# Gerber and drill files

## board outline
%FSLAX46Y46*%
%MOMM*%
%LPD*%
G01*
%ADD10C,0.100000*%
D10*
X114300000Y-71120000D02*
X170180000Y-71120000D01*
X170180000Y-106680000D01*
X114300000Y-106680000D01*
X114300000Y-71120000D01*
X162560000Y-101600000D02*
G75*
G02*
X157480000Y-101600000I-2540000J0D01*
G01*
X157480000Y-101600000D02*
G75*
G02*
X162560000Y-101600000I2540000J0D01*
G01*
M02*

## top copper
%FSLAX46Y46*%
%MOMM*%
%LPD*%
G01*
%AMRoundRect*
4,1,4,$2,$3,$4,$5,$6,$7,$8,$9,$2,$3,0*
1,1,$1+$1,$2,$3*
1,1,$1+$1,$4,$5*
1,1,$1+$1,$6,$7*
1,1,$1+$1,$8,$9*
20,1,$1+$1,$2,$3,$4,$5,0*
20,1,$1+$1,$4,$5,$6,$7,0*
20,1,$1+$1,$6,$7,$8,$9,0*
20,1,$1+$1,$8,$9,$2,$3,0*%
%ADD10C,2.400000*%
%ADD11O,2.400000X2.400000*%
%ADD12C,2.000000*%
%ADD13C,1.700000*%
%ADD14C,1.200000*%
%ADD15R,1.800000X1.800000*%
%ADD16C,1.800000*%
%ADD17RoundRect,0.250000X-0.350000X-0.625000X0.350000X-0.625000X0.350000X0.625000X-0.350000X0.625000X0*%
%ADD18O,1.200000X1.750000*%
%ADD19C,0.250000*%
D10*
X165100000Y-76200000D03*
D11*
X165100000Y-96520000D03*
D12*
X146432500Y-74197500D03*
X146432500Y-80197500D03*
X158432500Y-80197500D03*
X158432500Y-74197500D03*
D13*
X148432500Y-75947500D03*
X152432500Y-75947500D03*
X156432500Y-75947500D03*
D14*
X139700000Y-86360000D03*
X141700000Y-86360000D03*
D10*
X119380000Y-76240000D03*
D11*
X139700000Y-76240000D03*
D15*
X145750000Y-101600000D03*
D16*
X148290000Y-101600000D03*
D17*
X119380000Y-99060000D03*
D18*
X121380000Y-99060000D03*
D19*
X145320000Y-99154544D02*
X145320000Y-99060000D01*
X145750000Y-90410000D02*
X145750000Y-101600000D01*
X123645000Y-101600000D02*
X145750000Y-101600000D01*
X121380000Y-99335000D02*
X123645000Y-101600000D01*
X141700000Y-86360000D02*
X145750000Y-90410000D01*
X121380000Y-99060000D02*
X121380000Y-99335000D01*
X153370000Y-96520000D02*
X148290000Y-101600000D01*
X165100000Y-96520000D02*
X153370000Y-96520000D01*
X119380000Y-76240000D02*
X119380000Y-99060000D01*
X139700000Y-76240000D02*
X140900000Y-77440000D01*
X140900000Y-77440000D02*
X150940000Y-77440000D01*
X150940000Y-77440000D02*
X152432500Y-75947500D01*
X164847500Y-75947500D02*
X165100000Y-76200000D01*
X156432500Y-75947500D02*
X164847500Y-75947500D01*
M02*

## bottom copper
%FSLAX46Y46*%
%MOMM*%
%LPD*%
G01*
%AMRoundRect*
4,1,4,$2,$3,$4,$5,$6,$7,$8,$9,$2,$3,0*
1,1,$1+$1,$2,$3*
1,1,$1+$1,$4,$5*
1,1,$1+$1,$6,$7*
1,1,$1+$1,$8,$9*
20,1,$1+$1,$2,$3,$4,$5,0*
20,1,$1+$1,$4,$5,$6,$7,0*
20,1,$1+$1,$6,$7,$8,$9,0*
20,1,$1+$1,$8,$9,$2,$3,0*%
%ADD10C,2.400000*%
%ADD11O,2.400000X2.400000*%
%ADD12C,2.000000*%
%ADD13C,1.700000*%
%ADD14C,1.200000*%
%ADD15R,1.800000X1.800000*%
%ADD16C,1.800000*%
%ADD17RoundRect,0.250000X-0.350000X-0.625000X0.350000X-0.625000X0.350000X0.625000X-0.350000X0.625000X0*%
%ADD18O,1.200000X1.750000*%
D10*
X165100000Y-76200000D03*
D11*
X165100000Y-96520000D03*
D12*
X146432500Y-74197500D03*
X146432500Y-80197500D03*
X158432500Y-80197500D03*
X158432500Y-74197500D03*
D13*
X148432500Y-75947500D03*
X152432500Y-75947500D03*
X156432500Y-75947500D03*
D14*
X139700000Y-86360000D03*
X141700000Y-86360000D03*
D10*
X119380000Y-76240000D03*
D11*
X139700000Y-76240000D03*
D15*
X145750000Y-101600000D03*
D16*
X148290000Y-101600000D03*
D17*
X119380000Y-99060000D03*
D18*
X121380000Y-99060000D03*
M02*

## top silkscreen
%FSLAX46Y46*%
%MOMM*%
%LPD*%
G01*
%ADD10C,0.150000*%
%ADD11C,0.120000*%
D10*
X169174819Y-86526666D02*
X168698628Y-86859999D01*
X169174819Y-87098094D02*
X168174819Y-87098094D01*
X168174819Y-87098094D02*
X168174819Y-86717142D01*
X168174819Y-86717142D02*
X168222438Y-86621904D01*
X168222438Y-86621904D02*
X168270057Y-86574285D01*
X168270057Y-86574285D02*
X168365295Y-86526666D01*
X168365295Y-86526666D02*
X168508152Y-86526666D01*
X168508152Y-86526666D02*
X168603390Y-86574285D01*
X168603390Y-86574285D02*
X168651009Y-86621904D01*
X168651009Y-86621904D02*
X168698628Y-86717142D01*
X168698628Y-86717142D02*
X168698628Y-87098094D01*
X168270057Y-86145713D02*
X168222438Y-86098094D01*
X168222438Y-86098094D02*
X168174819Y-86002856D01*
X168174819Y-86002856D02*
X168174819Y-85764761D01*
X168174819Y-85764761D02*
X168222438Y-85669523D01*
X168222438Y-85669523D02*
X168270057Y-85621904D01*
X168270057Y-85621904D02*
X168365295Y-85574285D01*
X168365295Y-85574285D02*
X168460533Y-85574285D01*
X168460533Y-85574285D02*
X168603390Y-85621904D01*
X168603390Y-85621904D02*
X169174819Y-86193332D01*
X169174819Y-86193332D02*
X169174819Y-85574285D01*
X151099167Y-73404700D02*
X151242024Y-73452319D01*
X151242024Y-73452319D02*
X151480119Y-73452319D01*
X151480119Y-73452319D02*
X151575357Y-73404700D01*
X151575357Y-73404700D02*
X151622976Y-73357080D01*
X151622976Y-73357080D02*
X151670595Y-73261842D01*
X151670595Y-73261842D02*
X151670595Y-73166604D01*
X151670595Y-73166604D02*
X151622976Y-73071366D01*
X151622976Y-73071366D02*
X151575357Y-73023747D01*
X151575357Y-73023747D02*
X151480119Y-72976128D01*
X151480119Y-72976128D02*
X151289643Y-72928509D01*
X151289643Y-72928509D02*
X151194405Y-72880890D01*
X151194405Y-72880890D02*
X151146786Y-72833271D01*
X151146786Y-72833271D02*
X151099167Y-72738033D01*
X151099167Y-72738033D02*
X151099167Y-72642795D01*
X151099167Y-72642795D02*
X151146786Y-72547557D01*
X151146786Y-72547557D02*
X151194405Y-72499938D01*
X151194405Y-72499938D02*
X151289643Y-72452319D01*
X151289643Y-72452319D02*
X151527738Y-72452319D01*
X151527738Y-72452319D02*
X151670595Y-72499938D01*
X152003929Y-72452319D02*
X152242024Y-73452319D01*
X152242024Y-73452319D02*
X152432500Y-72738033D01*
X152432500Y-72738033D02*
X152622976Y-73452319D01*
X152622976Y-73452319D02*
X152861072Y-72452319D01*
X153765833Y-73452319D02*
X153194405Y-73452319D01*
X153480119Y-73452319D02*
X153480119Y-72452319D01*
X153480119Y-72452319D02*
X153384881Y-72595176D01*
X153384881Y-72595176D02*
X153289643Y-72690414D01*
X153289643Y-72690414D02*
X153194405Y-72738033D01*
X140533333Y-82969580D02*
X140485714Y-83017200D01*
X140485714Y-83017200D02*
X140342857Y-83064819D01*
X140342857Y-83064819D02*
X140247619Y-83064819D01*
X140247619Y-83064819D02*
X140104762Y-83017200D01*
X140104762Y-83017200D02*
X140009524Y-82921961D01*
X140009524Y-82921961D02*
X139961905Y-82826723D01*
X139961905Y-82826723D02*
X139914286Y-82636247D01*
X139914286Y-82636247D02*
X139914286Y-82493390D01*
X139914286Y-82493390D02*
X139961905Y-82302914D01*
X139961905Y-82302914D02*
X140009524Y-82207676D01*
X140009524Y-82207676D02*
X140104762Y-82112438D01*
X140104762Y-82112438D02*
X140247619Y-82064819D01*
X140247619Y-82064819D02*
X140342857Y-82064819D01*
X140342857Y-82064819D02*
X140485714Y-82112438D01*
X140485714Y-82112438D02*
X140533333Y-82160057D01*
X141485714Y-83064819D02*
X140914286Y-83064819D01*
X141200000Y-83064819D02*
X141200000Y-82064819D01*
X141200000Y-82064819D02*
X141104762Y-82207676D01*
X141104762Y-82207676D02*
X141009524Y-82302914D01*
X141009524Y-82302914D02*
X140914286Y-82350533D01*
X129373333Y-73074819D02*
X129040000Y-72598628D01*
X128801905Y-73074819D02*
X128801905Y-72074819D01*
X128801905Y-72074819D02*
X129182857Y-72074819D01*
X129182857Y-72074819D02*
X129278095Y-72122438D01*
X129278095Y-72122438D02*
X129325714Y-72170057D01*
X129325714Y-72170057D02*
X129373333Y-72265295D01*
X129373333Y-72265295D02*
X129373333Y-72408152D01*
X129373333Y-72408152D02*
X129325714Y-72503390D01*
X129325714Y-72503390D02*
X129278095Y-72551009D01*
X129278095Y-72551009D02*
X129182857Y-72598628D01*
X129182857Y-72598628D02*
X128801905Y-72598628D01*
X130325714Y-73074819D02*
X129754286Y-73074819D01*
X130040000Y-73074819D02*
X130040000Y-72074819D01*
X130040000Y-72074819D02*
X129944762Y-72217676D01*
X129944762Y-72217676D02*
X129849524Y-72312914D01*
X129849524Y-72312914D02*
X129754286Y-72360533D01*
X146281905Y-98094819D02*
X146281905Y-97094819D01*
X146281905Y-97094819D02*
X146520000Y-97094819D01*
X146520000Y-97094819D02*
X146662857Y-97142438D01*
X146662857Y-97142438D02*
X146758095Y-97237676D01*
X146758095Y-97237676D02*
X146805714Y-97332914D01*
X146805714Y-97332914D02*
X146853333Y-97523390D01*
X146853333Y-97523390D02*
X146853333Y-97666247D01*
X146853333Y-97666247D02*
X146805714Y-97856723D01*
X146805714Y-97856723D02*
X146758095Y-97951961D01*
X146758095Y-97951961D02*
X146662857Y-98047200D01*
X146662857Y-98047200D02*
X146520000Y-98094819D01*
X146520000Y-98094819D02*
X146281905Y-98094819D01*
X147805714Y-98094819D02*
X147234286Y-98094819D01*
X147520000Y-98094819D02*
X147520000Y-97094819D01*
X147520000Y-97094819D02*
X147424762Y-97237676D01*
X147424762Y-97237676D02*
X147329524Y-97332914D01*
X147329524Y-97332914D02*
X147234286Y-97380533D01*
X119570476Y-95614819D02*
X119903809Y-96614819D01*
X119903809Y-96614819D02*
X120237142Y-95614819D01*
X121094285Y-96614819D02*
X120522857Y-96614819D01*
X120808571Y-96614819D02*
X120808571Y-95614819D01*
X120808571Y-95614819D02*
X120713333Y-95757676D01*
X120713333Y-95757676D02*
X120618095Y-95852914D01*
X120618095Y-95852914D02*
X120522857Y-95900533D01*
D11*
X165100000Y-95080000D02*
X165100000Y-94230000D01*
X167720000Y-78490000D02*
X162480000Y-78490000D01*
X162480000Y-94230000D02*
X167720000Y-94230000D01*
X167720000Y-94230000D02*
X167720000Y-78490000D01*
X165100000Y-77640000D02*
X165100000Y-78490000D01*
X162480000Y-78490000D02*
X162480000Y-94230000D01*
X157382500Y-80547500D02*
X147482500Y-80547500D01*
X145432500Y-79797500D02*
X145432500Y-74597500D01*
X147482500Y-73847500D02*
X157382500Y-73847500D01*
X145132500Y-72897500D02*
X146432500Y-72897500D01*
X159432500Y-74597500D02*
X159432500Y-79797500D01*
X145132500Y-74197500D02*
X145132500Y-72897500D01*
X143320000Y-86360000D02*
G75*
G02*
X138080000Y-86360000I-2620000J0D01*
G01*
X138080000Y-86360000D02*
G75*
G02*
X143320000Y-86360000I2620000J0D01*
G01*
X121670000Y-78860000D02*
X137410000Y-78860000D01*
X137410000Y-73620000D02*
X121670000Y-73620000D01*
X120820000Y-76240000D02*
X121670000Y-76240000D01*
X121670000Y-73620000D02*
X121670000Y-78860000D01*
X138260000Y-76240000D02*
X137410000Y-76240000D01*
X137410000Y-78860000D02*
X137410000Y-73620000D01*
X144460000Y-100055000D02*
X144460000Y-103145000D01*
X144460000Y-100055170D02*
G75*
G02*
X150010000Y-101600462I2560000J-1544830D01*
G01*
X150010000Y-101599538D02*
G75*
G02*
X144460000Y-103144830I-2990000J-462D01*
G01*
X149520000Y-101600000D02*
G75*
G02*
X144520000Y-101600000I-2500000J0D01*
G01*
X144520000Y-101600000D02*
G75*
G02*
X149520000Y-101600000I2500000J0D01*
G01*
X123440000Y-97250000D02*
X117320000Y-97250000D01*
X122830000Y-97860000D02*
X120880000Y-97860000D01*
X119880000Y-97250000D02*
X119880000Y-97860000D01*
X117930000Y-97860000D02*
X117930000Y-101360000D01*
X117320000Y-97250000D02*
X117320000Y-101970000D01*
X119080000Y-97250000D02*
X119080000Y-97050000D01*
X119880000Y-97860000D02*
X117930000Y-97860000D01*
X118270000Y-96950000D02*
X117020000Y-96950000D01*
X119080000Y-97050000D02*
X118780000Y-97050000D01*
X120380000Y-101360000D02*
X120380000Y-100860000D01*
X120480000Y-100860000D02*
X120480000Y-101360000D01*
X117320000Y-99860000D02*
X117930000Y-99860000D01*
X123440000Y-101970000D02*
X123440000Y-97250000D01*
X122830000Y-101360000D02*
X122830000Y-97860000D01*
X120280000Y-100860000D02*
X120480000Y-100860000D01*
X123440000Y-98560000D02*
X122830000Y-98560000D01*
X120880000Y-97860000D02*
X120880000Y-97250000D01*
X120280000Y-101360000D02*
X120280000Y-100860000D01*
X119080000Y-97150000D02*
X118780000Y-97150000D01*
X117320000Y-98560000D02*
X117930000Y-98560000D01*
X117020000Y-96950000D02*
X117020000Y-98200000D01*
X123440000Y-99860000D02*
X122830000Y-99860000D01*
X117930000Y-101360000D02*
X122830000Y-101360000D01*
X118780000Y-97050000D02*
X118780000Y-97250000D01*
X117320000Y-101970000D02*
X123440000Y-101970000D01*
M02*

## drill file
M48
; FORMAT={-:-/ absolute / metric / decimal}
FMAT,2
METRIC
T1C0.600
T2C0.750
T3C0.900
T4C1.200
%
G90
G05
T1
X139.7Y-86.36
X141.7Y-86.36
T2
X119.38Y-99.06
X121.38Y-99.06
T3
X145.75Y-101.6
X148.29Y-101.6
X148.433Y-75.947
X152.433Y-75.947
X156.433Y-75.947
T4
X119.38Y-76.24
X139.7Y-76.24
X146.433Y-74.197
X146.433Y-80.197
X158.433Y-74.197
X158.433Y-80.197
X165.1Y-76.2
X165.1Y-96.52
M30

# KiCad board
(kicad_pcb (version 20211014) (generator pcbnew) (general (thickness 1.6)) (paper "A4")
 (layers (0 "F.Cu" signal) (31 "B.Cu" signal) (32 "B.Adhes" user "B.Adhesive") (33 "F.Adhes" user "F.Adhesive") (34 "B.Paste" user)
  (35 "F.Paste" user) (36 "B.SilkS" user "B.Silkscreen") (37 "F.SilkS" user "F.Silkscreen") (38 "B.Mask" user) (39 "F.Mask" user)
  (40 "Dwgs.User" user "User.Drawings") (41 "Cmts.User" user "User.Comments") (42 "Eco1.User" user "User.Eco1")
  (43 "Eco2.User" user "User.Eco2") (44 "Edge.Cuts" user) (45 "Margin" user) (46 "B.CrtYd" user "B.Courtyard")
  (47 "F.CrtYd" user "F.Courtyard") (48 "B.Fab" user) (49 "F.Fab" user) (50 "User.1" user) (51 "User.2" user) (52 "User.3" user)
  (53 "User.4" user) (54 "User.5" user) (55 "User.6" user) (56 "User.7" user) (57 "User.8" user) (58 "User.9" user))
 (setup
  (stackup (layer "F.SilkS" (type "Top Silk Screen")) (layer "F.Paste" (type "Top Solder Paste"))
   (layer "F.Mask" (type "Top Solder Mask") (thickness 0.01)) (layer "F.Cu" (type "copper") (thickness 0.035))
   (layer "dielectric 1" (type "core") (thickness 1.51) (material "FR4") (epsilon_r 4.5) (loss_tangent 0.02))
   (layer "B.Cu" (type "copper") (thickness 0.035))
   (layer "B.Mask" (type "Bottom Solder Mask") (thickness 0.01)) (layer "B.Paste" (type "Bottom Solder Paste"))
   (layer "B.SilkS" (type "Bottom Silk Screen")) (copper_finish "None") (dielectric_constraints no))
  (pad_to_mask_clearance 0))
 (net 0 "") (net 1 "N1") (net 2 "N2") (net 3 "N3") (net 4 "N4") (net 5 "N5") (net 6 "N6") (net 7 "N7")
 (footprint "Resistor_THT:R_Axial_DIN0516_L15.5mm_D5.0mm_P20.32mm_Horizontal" (layer "F.Cu") (at 165.1 76.2 -90)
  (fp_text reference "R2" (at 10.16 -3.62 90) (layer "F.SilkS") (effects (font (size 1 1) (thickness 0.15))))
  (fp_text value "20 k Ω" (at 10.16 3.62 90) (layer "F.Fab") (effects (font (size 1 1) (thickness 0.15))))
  (fp_line (start 18.88 0) (end 18.03 0) (layer "F.SilkS") (width 0.12))
  (fp_line (start 2.29 -2.62) (end 2.29 2.62) (layer "F.SilkS") (width 0.12))
  (fp_line (start 18.03 2.62) (end 18.03 -2.62) (layer "F.SilkS") (width 0.12))
  (fp_line (start 18.03 -2.62) (end 2.29 -2.62) (layer "F.SilkS") (width 0.12))
  (fp_line (start 1.44 0) (end 2.29 0) (layer "F.SilkS") (width 0.12))
  (fp_line (start 2.29 2.62) (end 18.03 2.62) (layer "F.SilkS") (width 0.12))
  (pad "1" thru_hole circle (at 0 0 270) (size 2.4 2.4) (drill 1.2) (layers *.Cu *.Mask) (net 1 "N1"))
  (pad "2" thru_hole oval (at 20.32 0 270) (size 2.4 2.4) (drill 1.2) (layers *.Cu *.Mask) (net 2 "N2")))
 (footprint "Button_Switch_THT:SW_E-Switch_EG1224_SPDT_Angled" (layer "F.Cu") (at 148.4325 75.9475)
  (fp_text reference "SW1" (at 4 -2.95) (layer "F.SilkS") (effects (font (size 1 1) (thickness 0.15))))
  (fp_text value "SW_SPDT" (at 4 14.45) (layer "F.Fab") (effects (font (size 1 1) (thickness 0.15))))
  (fp_line (start 8.95 4.6) (end -0.95 4.6) (layer "F.SilkS") (width 0.12))
  (fp_line (start -3 3.85) (end -3 -1.35) (layer "F.SilkS") (width 0.12))
  (fp_line (start -0.95 -2.1) (end 8.95 -2.1) (layer "F.SilkS") (width 0.12))
  (fp_line (start -3.3 -3.05) (end -2 -3.05) (layer "F.SilkS") (width 0.12))
  (fp_line (start 11 -1.35) (end 11 3.85) (layer "F.SilkS") (width 0.12))
  (fp_line (start -3.3 -1.75) (end -3.3 -3.05) (layer "F.SilkS") (width 0.12))
  (pad "" thru_hole circle (at -2 -1.75) (size 2 2) (drill 1.2) (layers *.Cu *.Mask))
  (pad "" thru_hole circle (at -2 4.25) (size 2 2) (drill 1.2) (layers *.Cu *.Mask))
  (pad "" thru_hole circle (at 10 4.25) (size 2 2) (drill 1.2) (layers *.Cu *.Mask))
  (pad "" thru_hole circle (at 10 -1.75) (size 2 2) (drill 1.2) (layers *.Cu *.Mask))
  (pad "1" thru_hole circle (at 0 0) (size 1.7 1.7) (drill 0.9) (layers *.Cu *.Mask) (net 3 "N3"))
  (pad "2" thru_hole circle (at 4 0) (size 1.7 1.7) (drill 0.9) (layers *.Cu *.Mask) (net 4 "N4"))
  (pad "3" thru_hole circle (at 8 0) (size 1.7 1.7) (drill 0.9) (layers *.Cu *.Mask) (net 1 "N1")))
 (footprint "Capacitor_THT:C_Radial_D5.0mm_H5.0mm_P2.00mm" (layer "F.Cu") (at 139.7 86.36)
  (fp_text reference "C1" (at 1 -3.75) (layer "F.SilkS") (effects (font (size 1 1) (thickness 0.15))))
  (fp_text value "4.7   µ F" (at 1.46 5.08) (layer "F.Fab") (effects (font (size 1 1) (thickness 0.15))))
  (fp_circle (center 1 0) (end 3.62 0) (layer "F.SilkS") (width 0.12) (fill none))
  (pad "1" thru_hole circle (at 0 0) (size 1.2 1.2) (drill 0.6) (layers *.Cu *.Mask) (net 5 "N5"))
  (pad "2" thru_hole circle (at 2 0) (size 1.2 1.2) (drill 0.6) (layers *.Cu *.Mask) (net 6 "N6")))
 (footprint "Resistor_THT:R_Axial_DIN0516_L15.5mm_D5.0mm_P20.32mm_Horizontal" (layer "F.Cu") (at 119.38 76.24)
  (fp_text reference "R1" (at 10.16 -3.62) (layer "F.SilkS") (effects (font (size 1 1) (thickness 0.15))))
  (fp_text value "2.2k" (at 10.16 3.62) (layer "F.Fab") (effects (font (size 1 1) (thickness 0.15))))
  (fp_line (start 2.29 2.62) (end 18.03 2.62) (layer "F.SilkS") (width 0.12))
  (fp_line (start 18.03 -2.62) (end 2.29 -2.62) (layer "F.SilkS") (width 0.12))
  (fp_line (start 1.44 0) (end 2.29 0) (layer "F.SilkS") (width 0.12))
  (fp_line (start 2.29 -2.62) (end 2.29 2.62) (layer "F.SilkS") (width 0.12))
  (fp_line (start 18.88 0) (end 18.03 0) (layer "F.SilkS") (width 0.12))
  (fp_line (start 18.03 2.62) (end 18.03 -2.62) (layer "F.SilkS") (width 0.12))
  (pad "1" thru_hole circle (at 0 0) (size 2.4 2.4) (drill 1.2) (layers *.Cu *.Mask) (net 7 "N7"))
  (pad "2" thru_hole oval (at 20.32 0) (size 2.4 2.4) (drill 1.2) (layers *.Cu *.Mask) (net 4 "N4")))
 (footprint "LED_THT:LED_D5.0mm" (layer "F.Cu") (at 145.75 101.6)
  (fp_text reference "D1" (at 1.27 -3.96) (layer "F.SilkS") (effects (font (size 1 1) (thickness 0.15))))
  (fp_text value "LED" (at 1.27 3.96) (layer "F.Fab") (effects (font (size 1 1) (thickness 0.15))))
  (fp_line (start -1.29 -1.545) (end -1.29 1.545) (layer "F.SilkS") (width 0.12))
  (fp_arc (start -1.29 -1.54483) (mid 2.072002 -2.880433) (end 4.26 0.000462) (layer "F.SilkS") (width 0.12))
  (fp_arc (start 4.26 -0.000462) (mid 2.072002 2.880433) (end -1.29 1.54483) (layer "F.SilkS") (width 0.12))
  (fp_circle (center 1.27 0) (end 3.77 0) (layer "F.SilkS") (width 0.12) (fill none))
  (pad "1" thru_hole rect (at 0 0) (size 1.8 1.8) (drill 0.9) (layers *.Cu *.Mask) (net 6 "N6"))
  (pad "2" thru_hole circle (at 2.54 0) (size 1.8 1.8) (drill 0.9) (layers *.Cu *.Mask) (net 2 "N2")))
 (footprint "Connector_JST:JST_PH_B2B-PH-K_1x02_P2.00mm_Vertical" (layer "F.Cu") (at 119.38 99.06)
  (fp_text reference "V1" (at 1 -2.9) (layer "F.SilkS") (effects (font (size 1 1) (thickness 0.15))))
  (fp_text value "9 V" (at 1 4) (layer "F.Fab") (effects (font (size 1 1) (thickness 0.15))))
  (fp_line (start 4.06 -1.81) (end -2.06 -1.81) (layer "F.SilkS") (width 0.12))
  (fp_line (start 3.45 -1.2) (end 1.5 -1.2) (layer "F.SilkS") (width 0.12))
  (fp_line (start 0.5 -1.81) (end 0.5 -1.2) (layer "F.SilkS") (width 0.12))
  (fp_line (start -1.45 -1.2) (end -1.45 2.3) (layer "F.SilkS") (width 0.12))
  (fp_line (start -2.06 -1.81) (end -2.06 2.91) (layer "F.SilkS") (width 0.12))
  (fp_line (start -0.3 -1.81) (end -0.3 -2.01) (layer "F.SilkS") (width 0.12))
  (fp_line (start 0.5 -1.2) (end -1.45 -1.2) (layer "F.SilkS") (width 0.12))
  (fp_line (start -1.11 -2.11) (end -2.36 -2.11) (layer "F.SilkS") (width 0.12))
  (fp_line (start -0.3 -2.01) (end -0.6 -2.01) (layer "F.SilkS") (width 0.12))
  (fp_line (start 1 2.3) (end 1 1.8) (layer "F.SilkS") (width 0.12))
  (fp_line (start 1.1 1.8) (end 1.1 2.3) (layer "F.SilkS") (width 0.12))
  (fp_line (start -2.06 0.8) (end -1.45 0.8) (layer "F.SilkS") (width 0.12))
  (fp_line (start 4.06 2.91) (end 4.06 -1.81) (layer "F.SilkS") (width 0.12))
  (fp_line (start 3.45 2.3) (end 3.45 -1.2) (layer "F.SilkS") (width 0.12))
  (fp_line (start 0.9 1.8) (end 1.1 1.8) (layer "F.SilkS") (width 0.12))
  (fp_line (start 4.06 -0.5) (end 3.45 -0.5) (layer "F.SilkS") (width 0.12))
  (fp_line (start 1.5 -1.2) (end 1.5 -1.81) (layer "F.SilkS") (width 0.12))
  (fp_line (start 0.9 2.3) (end 0.9 1.8) (layer "F.SilkS") (width 0.12))
  (fp_line (start -0.3 -1.91) (end -0.6 -1.91) (layer "F.SilkS") (width 0.12))
  (fp_line (start -2.06 -0.5) (end -1.45 -0.5) (layer "F.SilkS") (width 0.12))
  (fp_line (start -2.36 -2.11) (end -2.36 -0.86) (layer "F.SilkS") (width 0.12))
  (fp_line (start 4.06 0.8) (end 3.45 0.8) (layer "F.SilkS") (width 0.12))
  (fp_line (start -1.45 2.3) (end 3.45 2.3) (layer "F.SilkS") (width 0.12))
  (fp_line (start -0.6 -2.01) (end -0.6 -1.81) (layer "F.SilkS") (width 0.12))
  (fp_line (start -2.06 2.91) (end 4.06 2.91) (layer "F.SilkS") (width 0.12))
  (pad "1" thru_hole roundrect (at 0 0) (size 1.2 1.75) (drill 0.75) (layers *.Cu *.Mask) (roundrect_rratio 0.208333) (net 7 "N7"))
  (pad "2" thru_hole oval (at 2 0) (size 1.2 1.75) (drill 0.75) (layers *.Cu *.Mask) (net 6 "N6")))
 (gr_rect (start 114.3 71.12) (end 170.18 106.68) (layer "Edge.Cuts") (width 0.1) (fill none))
 (gr_circle (center 160.02 101.6) (end 162.56 101.6) (layer "Edge.Cuts") (width 0.1) (fill none))
 (segment (start 145.32 99.154544) (end 145.32 99.06) (width 0.25) (layer "F.Cu") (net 6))
 (segment (start 145.75 90.41) (end 145.75 101.6) (width 0.25) (layer "F.Cu") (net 6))
 (segment (start 123.645 101.6) (end 145.75 101.6) (width 0.25) (layer "F.Cu") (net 6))
 (segment (start 121.38 99.335) (end 123.645 101.6) (width 0.25) (layer "F.Cu") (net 6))
 (segment (start 141.7 86.36) (end 145.75 90.41) (width 0.25) (layer "F.Cu") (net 6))
 (segment (start 121.38 99.06) (end 121.38 99.335) (width 0.25) (layer "F.Cu") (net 6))
 (segment (start 153.37 96.52) (end 148.29 101.6) (width 0.25) (layer "F.Cu") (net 2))
 (segment (start 165.1 96.52) (end 153.37 96.52) (width 0.25) (layer "F.Cu") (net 2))
 (segment (start 119.38 76.24) (end 119.38 99.06) (width 0.25) (layer "F.Cu") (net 7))
 (segment (start 139.7 76.24) (end 140.9 77.44) (width 0.25) (layer "F.Cu") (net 4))
 (segment (start 140.9 77.44) (end 150.94 77.44) (width 0.25) (layer "F.Cu") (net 4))
 (segment (start 150.94 77.44) (end 152.4325 75.9475) (width 0.25) (layer "F.Cu") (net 4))
 (segment (start 164.8475 75.9475) (end 165.1 76.2) (width 0.25) (layer "F.Cu") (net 1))
 (segment (start 156.4325 75.9475) (end 164.8475 75.9475) (width 0.25) (layer "F.Cu") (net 1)))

